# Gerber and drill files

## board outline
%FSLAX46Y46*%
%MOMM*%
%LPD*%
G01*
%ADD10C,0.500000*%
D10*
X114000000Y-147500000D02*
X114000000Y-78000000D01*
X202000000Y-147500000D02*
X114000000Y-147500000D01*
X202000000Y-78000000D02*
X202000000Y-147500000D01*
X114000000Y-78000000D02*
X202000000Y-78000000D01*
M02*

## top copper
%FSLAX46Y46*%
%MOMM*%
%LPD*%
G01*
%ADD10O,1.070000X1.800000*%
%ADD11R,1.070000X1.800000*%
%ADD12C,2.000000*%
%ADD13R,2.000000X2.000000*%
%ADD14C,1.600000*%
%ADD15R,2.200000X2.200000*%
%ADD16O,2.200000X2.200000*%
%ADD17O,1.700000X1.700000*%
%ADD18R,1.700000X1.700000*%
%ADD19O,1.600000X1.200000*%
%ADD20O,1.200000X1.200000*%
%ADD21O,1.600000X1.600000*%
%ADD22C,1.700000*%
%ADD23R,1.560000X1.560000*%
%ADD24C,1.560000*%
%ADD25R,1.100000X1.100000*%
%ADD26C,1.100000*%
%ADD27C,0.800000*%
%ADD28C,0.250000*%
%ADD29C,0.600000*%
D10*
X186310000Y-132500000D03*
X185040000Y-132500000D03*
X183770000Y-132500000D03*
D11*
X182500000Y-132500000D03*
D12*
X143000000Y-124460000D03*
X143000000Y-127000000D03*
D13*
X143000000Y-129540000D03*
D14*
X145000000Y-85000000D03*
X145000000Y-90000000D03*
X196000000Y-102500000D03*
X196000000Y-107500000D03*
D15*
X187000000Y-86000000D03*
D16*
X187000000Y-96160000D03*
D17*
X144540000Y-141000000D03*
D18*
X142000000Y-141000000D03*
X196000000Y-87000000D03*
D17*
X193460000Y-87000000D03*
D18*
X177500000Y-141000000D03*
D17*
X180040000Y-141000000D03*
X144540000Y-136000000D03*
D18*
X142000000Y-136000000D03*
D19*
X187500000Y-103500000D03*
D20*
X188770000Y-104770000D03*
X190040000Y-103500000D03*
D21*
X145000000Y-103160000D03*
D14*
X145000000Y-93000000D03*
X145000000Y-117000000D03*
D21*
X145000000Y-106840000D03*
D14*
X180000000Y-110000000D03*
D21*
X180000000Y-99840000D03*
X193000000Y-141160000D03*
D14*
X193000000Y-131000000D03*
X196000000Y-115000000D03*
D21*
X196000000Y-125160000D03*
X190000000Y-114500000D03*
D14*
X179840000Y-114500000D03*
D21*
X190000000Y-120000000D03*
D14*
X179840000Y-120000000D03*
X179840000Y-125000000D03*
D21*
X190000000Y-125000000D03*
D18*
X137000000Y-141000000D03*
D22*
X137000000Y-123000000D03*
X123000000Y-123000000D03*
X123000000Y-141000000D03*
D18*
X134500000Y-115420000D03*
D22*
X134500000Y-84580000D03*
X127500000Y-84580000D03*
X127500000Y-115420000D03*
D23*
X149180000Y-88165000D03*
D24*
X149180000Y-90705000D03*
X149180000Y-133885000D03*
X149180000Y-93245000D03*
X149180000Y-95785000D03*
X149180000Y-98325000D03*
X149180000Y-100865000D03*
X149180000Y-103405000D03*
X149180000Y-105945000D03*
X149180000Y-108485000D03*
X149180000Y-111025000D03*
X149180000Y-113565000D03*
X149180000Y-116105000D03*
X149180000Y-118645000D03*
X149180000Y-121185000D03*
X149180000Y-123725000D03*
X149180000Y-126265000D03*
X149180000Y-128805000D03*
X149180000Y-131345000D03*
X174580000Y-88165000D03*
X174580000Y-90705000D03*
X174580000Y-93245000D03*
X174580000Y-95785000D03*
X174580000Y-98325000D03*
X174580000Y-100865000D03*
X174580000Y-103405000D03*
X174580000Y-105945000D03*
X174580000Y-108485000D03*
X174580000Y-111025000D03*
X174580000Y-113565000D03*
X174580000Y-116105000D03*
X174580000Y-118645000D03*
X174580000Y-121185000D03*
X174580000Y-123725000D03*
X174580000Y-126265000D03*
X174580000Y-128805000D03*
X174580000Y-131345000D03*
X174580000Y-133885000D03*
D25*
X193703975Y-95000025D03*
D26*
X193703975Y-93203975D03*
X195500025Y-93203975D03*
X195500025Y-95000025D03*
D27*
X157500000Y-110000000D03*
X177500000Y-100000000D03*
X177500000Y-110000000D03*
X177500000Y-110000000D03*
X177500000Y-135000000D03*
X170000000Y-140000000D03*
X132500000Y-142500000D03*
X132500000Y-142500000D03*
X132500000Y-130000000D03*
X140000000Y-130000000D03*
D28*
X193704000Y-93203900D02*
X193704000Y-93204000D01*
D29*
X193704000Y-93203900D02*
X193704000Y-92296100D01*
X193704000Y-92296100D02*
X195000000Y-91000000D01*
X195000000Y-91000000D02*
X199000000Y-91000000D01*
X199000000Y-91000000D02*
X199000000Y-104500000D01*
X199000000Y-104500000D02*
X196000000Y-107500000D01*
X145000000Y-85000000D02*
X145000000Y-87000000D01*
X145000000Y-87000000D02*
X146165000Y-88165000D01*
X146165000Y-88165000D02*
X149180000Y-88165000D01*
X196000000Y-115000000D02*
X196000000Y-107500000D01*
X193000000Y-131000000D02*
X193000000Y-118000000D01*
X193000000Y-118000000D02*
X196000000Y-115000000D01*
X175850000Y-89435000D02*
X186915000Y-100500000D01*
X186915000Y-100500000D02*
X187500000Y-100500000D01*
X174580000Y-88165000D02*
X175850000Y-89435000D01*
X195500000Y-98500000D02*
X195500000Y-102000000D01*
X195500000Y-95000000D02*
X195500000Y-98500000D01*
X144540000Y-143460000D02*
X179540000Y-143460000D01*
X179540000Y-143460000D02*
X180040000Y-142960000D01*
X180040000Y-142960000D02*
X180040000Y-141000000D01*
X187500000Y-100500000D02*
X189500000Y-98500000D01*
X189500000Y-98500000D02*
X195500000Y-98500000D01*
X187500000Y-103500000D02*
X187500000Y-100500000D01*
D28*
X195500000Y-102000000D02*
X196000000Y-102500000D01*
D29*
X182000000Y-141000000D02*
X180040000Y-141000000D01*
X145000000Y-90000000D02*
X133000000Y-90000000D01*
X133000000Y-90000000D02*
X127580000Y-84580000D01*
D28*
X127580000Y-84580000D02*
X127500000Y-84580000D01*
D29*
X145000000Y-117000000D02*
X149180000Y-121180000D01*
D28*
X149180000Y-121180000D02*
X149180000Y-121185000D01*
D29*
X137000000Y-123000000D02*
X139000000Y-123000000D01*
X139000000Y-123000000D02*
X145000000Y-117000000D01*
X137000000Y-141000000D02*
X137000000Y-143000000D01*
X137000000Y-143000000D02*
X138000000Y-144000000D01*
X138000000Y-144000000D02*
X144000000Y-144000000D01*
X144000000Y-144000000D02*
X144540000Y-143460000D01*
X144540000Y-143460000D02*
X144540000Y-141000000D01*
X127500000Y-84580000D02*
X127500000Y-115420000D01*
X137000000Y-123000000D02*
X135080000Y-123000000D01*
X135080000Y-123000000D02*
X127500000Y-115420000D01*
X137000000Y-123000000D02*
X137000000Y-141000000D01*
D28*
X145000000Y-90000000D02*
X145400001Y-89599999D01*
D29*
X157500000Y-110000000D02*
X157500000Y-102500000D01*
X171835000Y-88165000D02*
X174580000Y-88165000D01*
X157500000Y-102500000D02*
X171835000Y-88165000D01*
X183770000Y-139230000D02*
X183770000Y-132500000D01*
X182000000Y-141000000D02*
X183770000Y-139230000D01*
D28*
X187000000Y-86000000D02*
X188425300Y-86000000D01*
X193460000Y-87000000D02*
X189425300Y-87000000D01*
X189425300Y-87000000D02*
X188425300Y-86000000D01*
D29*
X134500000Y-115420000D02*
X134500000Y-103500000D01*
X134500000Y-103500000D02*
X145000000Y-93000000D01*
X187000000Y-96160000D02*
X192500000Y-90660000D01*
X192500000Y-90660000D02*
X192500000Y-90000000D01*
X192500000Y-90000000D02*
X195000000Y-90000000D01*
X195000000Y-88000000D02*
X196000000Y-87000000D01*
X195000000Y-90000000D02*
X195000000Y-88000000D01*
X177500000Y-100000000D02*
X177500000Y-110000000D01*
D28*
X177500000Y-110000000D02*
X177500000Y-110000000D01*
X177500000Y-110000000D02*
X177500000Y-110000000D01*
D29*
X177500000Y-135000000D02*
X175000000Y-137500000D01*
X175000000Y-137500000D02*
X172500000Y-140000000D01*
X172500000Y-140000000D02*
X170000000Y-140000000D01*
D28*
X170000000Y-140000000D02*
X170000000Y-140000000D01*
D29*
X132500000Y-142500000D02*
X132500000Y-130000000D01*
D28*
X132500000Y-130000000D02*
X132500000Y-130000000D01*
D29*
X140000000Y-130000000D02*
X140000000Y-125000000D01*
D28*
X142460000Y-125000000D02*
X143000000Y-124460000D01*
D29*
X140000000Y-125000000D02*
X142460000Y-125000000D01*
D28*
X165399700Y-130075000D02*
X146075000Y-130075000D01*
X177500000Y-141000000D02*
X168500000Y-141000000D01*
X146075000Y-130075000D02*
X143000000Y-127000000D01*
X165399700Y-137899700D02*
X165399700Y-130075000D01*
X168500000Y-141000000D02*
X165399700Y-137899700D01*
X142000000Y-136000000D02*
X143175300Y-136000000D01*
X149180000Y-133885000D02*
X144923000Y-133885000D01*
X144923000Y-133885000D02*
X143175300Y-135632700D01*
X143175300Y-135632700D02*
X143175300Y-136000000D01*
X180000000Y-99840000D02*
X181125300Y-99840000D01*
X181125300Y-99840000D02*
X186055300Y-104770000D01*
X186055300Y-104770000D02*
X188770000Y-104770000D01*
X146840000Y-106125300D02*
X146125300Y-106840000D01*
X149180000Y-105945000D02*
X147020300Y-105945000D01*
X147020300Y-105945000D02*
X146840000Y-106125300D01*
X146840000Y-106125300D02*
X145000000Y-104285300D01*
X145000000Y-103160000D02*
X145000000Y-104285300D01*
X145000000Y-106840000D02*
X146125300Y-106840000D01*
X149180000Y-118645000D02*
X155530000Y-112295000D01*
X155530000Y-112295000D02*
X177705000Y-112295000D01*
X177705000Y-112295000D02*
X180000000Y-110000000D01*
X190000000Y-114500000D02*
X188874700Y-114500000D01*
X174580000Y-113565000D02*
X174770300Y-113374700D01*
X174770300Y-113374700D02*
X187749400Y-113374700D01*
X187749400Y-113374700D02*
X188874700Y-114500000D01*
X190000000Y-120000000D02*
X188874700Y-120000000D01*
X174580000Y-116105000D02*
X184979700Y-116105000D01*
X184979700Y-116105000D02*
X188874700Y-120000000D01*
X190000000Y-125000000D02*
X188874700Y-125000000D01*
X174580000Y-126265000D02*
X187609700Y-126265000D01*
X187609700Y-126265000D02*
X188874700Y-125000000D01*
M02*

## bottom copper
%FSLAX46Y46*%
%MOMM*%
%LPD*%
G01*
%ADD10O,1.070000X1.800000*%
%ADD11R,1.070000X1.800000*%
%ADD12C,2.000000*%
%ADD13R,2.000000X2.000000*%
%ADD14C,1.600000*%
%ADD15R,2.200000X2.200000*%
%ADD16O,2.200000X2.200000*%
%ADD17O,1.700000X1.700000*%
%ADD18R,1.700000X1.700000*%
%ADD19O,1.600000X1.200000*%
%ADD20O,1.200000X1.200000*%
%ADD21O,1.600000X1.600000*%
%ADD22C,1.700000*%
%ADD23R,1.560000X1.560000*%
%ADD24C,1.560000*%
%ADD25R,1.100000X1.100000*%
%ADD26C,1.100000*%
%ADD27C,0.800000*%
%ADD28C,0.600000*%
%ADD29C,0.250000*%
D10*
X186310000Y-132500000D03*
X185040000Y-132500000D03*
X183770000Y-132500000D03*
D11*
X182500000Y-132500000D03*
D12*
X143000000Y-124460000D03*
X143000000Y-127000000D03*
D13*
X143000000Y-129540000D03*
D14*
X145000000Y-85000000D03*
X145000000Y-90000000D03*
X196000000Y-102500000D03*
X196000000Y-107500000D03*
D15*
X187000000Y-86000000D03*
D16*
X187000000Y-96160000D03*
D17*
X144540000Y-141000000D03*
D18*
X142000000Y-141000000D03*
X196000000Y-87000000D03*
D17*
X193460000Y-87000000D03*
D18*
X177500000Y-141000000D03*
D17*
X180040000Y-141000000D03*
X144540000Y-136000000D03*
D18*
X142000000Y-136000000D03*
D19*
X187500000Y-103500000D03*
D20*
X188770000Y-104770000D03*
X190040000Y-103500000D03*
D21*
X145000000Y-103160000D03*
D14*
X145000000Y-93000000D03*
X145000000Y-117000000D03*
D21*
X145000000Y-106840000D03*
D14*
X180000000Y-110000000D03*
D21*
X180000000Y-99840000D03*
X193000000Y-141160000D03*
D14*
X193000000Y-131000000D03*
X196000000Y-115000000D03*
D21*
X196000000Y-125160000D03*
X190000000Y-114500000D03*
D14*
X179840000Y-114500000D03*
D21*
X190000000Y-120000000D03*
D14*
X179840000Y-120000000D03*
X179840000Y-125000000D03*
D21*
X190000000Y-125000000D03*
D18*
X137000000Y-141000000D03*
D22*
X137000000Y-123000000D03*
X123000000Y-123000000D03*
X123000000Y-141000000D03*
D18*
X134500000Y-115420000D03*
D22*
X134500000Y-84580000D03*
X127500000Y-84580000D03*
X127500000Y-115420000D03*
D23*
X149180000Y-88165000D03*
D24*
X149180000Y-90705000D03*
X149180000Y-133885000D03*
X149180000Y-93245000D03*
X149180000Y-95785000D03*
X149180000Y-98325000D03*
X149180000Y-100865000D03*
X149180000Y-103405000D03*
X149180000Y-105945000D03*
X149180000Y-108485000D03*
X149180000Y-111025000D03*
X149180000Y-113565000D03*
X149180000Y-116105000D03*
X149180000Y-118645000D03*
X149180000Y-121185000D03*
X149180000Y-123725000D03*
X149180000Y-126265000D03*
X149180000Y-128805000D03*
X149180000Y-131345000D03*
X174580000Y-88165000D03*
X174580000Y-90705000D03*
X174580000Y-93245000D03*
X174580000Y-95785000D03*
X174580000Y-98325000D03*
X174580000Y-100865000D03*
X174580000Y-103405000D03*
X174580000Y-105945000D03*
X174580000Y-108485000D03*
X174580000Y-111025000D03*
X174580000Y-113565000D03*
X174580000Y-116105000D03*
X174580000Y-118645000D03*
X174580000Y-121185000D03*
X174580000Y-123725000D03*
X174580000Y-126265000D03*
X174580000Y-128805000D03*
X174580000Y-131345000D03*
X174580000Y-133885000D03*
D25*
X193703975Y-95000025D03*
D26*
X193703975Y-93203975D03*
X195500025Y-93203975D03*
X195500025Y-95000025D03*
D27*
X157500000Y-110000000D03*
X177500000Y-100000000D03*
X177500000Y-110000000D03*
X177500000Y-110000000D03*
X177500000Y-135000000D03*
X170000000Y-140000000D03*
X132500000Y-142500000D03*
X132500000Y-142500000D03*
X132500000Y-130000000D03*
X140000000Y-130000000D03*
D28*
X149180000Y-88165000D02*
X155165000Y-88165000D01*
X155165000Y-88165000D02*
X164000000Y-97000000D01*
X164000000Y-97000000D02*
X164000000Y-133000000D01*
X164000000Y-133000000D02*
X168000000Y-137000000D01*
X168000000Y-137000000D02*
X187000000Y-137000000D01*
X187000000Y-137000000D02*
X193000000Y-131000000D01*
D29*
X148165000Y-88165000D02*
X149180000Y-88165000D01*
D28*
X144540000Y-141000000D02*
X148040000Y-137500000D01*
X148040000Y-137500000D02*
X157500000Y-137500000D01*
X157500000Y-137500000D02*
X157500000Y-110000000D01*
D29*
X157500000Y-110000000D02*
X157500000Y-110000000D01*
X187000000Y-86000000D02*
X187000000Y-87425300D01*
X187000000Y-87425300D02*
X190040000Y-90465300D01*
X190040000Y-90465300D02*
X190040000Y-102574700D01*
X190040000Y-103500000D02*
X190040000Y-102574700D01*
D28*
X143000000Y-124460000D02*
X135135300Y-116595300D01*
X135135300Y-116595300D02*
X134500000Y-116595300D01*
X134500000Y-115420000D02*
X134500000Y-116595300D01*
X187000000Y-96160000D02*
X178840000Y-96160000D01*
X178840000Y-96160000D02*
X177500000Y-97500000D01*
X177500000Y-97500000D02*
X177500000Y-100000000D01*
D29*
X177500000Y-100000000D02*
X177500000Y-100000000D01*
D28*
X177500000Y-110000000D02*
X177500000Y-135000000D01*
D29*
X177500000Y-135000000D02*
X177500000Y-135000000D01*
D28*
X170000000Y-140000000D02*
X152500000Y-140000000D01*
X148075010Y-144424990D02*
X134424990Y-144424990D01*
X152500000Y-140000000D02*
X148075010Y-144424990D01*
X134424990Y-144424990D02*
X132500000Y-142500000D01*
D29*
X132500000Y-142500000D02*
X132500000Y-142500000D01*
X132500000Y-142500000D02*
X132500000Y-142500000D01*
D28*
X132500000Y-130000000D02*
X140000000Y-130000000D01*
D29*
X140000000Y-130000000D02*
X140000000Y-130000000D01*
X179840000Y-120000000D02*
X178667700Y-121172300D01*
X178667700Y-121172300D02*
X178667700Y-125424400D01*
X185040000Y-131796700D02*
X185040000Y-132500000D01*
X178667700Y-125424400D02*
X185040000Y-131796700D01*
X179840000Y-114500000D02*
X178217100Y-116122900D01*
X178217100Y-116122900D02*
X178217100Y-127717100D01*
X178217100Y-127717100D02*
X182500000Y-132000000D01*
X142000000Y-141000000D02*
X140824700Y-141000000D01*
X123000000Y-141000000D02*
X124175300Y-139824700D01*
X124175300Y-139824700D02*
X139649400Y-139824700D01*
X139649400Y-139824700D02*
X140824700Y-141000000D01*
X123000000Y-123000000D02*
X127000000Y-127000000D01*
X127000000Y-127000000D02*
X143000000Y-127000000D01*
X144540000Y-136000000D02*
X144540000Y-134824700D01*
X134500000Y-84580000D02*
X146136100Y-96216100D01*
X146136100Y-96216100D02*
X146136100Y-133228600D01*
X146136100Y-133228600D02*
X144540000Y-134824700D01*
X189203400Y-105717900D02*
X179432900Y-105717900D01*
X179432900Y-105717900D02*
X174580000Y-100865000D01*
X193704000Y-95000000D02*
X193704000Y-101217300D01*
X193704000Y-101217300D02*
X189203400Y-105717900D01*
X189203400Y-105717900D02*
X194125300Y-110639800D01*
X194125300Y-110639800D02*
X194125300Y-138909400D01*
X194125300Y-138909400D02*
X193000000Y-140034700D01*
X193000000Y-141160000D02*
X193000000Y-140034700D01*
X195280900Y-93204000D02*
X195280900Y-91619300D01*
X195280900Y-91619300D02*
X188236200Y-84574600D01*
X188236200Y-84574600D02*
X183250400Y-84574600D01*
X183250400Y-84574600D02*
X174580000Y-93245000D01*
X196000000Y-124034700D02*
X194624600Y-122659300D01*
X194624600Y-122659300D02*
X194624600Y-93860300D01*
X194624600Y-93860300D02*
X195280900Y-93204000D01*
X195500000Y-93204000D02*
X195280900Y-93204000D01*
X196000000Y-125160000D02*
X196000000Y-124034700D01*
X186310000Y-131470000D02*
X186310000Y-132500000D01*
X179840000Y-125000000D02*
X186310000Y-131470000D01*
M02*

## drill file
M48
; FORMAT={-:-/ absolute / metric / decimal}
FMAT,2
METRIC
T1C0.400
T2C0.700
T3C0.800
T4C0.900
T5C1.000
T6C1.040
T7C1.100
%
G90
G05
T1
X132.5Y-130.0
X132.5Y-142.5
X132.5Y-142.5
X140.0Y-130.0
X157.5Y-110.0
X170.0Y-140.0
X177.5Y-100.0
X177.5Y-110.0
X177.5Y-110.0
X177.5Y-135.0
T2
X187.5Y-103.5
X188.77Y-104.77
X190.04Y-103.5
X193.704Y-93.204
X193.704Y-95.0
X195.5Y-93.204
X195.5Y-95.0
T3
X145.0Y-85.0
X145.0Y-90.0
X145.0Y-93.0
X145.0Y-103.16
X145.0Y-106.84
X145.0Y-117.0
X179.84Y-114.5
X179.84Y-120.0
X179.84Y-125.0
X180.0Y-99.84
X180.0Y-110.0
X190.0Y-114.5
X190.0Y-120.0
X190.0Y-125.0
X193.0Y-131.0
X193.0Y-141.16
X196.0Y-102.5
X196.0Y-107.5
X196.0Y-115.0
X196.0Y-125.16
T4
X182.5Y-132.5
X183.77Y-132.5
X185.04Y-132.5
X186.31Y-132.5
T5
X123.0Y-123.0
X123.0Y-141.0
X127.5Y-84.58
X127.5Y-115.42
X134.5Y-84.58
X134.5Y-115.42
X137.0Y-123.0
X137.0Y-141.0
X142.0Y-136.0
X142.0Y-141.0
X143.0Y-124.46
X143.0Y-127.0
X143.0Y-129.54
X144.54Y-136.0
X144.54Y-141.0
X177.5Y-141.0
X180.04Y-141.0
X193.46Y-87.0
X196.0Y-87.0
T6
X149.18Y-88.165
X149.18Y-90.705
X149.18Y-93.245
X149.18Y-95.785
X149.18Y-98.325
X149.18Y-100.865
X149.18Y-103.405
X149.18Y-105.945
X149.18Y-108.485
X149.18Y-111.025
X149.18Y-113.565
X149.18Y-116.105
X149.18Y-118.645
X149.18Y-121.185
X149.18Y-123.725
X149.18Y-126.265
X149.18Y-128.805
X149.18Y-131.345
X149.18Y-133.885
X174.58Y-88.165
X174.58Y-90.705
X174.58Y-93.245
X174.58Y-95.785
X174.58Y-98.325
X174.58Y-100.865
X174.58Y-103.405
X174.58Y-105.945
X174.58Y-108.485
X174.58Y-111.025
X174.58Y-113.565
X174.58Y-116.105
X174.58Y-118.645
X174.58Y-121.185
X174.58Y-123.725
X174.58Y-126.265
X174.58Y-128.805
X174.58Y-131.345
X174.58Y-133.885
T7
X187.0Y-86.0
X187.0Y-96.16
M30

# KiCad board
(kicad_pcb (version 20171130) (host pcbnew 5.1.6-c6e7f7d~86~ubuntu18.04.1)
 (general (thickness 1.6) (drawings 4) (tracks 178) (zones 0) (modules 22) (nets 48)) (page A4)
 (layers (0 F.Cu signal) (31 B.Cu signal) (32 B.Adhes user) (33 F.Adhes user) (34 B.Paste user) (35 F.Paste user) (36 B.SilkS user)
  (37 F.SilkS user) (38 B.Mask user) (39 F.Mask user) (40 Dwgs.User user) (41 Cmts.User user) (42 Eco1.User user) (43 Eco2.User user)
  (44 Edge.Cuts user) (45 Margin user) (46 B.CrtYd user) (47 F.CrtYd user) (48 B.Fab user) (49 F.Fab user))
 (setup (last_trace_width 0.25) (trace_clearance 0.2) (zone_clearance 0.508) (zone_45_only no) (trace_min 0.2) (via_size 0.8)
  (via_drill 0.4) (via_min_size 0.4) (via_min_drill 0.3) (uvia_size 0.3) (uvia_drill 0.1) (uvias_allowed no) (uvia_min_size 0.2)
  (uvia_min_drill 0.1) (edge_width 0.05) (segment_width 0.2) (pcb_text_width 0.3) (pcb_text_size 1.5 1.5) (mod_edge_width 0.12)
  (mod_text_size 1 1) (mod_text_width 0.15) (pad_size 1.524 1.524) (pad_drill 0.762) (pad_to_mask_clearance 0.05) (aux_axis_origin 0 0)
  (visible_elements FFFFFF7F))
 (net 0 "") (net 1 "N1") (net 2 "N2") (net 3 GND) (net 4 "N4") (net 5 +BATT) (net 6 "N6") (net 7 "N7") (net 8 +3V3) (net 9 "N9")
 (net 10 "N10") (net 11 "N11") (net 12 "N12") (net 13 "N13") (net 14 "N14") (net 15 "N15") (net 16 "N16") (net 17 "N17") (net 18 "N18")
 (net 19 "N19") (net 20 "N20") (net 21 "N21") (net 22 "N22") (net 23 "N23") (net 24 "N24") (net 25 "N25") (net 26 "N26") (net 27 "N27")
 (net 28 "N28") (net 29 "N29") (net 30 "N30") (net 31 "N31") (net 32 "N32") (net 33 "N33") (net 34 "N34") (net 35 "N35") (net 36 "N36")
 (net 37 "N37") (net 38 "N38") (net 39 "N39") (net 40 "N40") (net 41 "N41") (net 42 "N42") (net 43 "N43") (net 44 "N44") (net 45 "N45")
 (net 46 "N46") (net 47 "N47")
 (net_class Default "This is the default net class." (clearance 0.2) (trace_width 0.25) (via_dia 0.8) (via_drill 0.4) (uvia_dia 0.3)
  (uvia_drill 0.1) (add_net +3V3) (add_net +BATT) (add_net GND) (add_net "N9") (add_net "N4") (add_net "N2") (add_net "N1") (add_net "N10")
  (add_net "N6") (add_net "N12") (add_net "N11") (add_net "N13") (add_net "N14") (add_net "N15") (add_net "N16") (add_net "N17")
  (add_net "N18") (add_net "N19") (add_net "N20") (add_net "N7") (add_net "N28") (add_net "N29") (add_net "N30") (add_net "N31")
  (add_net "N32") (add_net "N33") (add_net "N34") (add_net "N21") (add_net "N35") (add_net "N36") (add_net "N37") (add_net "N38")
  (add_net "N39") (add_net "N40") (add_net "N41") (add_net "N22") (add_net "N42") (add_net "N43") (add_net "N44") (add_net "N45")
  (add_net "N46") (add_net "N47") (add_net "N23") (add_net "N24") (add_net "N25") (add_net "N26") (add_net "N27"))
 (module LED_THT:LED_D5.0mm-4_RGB (layer F.Cu) (at 182.5 132.5)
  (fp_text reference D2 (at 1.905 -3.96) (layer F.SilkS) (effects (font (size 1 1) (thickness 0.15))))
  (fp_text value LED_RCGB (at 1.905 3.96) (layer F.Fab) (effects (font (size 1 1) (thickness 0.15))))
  (pad 4 thru_hole oval (at 3.81 0) (size 1.07 1.8) (drill 0.9) (layers *.Cu *.Mask) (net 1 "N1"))
  (pad 3 thru_hole oval (at 2.54 0) (size 1.07 1.8) (drill 0.9) (layers *.Cu *.Mask) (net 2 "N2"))
  (pad 2 thru_hole oval (at 1.27 0) (size 1.07 1.8) (drill 0.9) (layers *.Cu *.Mask) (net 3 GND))
  (pad 1 thru_hole rect (at 0 0) (size 1.07 1.8) (drill 0.9) (layers *.Cu *.Mask) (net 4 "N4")))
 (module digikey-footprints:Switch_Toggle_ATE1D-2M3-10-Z (layer F.Cu) (at 143 127 90)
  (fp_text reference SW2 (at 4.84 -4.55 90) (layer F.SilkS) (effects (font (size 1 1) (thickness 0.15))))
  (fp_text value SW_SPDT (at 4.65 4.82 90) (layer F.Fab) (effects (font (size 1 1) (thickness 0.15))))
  (pad 3 thru_hole circle (at 2.54 0 90) (size 2 2) (drill 1) (layers *.Cu *.Mask) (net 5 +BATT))
  (pad 2 thru_hole circle (at 0 0 90) (size 2 2) (drill 1) (layers *.Cu *.Mask) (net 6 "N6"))
  (pad 1 thru_hole rect (at -2.54 0 90) (size 2 2) (drill 1) (layers *.Cu *.Mask) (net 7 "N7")))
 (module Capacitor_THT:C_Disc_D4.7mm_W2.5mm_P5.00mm (layer F.Cu) (at 145 85 270)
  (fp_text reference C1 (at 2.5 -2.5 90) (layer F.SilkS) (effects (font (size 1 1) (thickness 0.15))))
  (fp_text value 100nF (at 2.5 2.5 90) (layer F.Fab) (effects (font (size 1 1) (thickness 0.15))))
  (pad 1 thru_hole circle (at 0 0 270) (size 1.6 1.6) (drill 0.8) (layers *.Cu *.Mask) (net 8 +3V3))
  (pad 2 thru_hole circle (at 5 0 270) (size 1.6 1.6) (drill 0.8) (layers *.Cu *.Mask) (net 3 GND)))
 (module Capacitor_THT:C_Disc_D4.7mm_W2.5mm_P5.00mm (layer F.Cu) (at 196 107.5 90)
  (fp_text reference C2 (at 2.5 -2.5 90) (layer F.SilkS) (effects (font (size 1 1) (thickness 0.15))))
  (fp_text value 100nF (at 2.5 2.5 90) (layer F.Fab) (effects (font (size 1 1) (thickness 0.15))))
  (pad 2 thru_hole circle (at 5 0 90) (size 1.6 1.6) (drill 0.8) (layers *.Cu *.Mask) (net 3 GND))
  (pad 1 thru_hole circle (at 0 0 90) (size 1.6 1.6) (drill 0.8) (layers *.Cu *.Mask) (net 8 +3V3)))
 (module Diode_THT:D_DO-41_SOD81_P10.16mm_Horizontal (layer F.Cu) (at 187 86 270)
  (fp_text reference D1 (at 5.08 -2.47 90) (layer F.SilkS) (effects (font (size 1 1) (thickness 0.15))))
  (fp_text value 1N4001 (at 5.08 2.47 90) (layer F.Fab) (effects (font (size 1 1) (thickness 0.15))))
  (pad 1 thru_hole rect (at 0 0 270) (size 2.2 2.2) (drill 1.1) (layers *.Cu *.Mask) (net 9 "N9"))
  (pad 2 thru_hole oval (at 10.16 0 270) (size 2.2 2.2) (drill 1.1) (layers *.Cu *.Mask) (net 5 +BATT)))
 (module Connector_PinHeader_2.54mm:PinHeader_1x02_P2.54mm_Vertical (layer F.Cu) (at 142 141 90)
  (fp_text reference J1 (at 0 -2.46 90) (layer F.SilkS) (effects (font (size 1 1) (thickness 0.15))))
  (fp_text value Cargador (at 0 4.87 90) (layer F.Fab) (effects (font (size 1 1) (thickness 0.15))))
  (pad 2 thru_hole oval (at 0 2.54 90) (size 1.7 1.7) (drill 1) (layers *.Cu *.Mask) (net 3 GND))
  (pad 1 thru_hole rect (at 0 0 90) (size 1.7 1.7) (drill 1) (layers *.Cu *.Mask) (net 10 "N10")))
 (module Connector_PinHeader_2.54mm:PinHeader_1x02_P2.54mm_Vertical (layer F.Cu) (at 196 87 270)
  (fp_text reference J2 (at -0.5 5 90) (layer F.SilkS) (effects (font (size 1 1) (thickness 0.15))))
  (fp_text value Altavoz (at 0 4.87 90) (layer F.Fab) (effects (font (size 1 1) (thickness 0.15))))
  (pad 1 thru_hole rect (at 0 0 270) (size 1.7 1.7) (drill 1) (layers *.Cu *.Mask) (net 5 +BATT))
  (pad 2 thru_hole oval (at 0 2.54 270) (size 1.7 1.7) (drill 1) (layers *.Cu *.Mask) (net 9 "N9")))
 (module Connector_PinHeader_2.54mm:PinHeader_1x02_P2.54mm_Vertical (layer F.Cu) (at 177.5 141 90)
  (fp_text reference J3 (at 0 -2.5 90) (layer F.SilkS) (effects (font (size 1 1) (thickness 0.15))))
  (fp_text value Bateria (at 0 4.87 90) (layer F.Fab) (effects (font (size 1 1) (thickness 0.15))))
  (pad 1 thru_hole rect (at 0 0 90) (size 1.7 1.7) (drill 1) (layers *.Cu *.Mask) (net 6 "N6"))
  (pad 2 thru_hole oval (at 0 2.54 90) (size 1.7 1.7) (drill 1) (layers *.Cu *.Mask) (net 3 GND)))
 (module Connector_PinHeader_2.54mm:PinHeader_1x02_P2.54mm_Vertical (layer F.Cu) (at 142 136 90)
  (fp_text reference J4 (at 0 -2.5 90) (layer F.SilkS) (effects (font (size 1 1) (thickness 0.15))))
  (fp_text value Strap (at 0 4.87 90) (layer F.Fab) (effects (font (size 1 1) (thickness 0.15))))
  (pad 2 thru_hole oval (at 0 2.54 90) (size 1.7 1.7) (drill 1) (layers *.Cu *.Mask) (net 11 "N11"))
  (pad 1 thru_hole rect (at 0 0 90) (size 1.7 1.7) (drill 1) (layers *.Cu *.Mask) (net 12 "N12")))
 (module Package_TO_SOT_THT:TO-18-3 (layer F.Cu) (at 187.5 103.5)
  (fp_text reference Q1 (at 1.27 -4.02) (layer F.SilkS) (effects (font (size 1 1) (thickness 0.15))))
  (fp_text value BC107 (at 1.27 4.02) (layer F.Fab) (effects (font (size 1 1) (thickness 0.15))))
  (pad 1 thru_hole oval (at 0 0) (size 1.6 1.2) (drill 0.7) (layers *.Cu *.Mask) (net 3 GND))
  (pad 2 thru_hole oval (at 1.27 1.27) (size 1.2 1.2) (drill 0.7) (layers *.Cu *.Mask) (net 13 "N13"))
  (pad 3 thru_hole oval (at 2.54 0) (size 1.2 1.2) (drill 0.7) (layers *.Cu *.Mask) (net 9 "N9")))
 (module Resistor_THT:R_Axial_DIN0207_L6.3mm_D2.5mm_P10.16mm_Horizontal (layer F.Cu) (at 145 93 270)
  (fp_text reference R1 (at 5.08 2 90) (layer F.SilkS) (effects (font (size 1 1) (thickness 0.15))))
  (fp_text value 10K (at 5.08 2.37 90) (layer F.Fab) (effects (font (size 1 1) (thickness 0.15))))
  (pad 2 thru_hole oval (at 10.16 0 270) (size 1.6 1.6) (drill 0.8) (layers *.Cu *.Mask) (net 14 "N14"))
  (pad 1 thru_hole circle (at 0 0 270) (size 1.6 1.6) (drill 0.8) (layers *.Cu *.Mask) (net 5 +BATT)))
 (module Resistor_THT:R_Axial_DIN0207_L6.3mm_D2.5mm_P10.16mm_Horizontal (layer F.Cu) (at 145 117 90)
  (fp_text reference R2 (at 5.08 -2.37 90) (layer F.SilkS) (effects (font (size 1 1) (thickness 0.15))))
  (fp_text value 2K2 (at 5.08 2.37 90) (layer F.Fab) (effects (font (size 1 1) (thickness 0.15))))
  (pad 1 thru_hole circle (at 0 0 90) (size 1.6 1.6) (drill 0.8) (layers *.Cu *.Mask) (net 3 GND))
  (pad 2 thru_hole oval (at 10.16 0 90) (size 1.6 1.6) (drill 0.8) (layers *.Cu *.Mask) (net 14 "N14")))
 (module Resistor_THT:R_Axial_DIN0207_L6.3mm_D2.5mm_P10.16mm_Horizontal (layer F.Cu) (at 180 110 90)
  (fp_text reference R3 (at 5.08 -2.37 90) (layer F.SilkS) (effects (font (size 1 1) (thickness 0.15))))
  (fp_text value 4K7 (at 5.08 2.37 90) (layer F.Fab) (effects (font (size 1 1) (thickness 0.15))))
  (pad 1 thru_hole circle (at 0 0 90) (size 1.6 1.6) (drill 0.8) (layers *.Cu *.Mask) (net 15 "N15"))
  (pad 2 thru_hole oval (at 10.16 0 90) (size 1.6 1.6) (drill 0.8) (layers *.Cu *.Mask) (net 13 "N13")))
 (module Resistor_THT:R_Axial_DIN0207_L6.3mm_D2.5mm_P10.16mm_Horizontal (layer F.Cu) (at 193 131 270)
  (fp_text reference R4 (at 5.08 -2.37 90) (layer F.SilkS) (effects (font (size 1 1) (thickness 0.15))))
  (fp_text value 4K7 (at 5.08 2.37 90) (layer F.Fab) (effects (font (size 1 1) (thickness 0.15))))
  (pad 2 thru_hole oval (at 10.16 0 270) (size 1.6 1.6) (drill 0.8) (layers *.Cu *.Mask) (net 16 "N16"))
  (pad 1 thru_hole circle (at 0 0 270) (size 1.6 1.6) (drill 0.8) (layers *.Cu *.Mask) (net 8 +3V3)))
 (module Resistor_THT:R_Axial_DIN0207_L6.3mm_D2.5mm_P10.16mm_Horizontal (layer F.Cu) (at 196 115 270)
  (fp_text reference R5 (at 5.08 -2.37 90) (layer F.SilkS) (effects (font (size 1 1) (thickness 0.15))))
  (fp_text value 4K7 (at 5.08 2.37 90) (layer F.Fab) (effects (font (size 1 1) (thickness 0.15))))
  (pad 1 thru_hole circle (at 0 0 270) (size 1.6 1.6) (drill 0.8) (layers *.Cu *.Mask) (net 8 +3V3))
  (pad 2 thru_hole oval (at 10.16 0 270) (size 1.6 1.6) (drill 0.8) (layers *.Cu *.Mask) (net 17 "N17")))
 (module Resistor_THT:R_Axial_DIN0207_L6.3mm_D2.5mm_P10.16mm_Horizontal (layer F.Cu) (at 179.84 114.5)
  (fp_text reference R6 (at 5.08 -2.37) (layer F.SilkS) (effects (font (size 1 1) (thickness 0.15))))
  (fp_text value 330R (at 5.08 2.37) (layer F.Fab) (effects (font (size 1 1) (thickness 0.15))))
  (pad 2 thru_hole oval (at 10.16 0) (size 1.6 1.6) (drill 0.8) (layers *.Cu *.Mask) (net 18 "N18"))
  (pad 1 thru_hole circle (at 0 0) (size 1.6 1.6) (drill 0.8) (layers *.Cu *.Mask) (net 4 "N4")))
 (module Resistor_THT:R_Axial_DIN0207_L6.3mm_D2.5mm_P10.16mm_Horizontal (layer F.Cu) (at 179.84 120)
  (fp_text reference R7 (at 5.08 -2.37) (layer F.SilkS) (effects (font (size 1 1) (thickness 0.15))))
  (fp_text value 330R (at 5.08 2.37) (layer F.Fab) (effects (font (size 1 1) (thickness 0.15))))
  (pad 2 thru_hole oval (at 10.16 0) (size 1.6 1.6) (drill 0.8) (layers *.Cu *.Mask) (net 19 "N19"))
  (pad 1 thru_hole circle (at 0 0) (size 1.6 1.6) (drill 0.8) (layers *.Cu *.Mask) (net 2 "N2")))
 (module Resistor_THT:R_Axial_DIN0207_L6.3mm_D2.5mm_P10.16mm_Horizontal (layer F.Cu) (at 179.84 125)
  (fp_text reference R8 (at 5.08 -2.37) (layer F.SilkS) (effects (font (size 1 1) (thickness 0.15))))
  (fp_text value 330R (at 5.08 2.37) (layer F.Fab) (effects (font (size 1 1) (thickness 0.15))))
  (pad 1 thru_hole circle (at 0 0) (size 1.6 1.6) (drill 0.8) (layers *.Cu *.Mask) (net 1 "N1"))
  (pad 2 thru_hole oval (at 10.16 0) (size 1.6 1.6) (drill 0.8) (layers *.Cu *.Mask) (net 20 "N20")))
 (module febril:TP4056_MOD (layer F.Cu) (at 130 132 90)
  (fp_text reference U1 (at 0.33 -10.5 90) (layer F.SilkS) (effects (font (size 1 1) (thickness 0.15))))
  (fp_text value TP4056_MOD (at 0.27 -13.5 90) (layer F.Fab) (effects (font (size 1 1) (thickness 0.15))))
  (pad 1 thru_hole rect (at -9 7 90) (size 1.7 1.7) (drill 1) (layers *.Cu *.Mask) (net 3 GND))
  (pad 2 thru_hole circle (at 9 7 90) (size 1.7 1.7) (drill 1) (layers *.Cu *.Mask) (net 3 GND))
  (pad 3 thru_hole circle (at 9 -7 90) (size 1.7 1.7) (drill 1) (layers *.Cu *.Mask) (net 6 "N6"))
  (pad 4 thru_hole circle (at -9 -7 90) (size 1.7 1.7) (drill 1) (layers *.Cu *.Mask) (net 10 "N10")))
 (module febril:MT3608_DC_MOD (layer F.Cu) (at 131 100 90)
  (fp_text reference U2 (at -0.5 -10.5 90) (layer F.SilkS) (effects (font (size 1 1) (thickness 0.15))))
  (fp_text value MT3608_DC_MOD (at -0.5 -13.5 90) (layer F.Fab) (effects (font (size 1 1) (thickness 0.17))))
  (pad 1 thru_hole rect (at -15.42 3.5 90) (size 1.7 1.7) (drill 1) (layers *.Cu *.Mask) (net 5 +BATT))
  (pad 2 thru_hole circle (at 15.42 3.5 90) (size 1.7 1.7) (drill 1) (layers *.Cu *.Mask) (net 11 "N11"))
  (pad 3 thru_hole circle (at 15.42 -3.5 90) (size 1.7 1.7) (drill 1) (layers *.Cu *.Mask) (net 3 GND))
  (pad 4 thru_hole circle (at -15.42 -3.5 90) (size 1.7 1.7) (drill 1) (layers *.Cu *.Mask) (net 3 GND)))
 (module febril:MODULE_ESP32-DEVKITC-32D (layer F.Cu) (at 161.88 107.925)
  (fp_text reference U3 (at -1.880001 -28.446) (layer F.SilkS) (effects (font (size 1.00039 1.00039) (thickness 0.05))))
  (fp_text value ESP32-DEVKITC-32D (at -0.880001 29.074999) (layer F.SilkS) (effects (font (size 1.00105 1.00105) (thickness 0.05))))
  (pad 1 thru_hole rect (at -12.7 -19.76) (size 1.56 1.56) (drill 1.04) (layers *.Cu *.Mask) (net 8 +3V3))
  (pad 2 thru_hole circle (at -12.7 -17.22) (size 1.56 1.56) (drill 1.04) (layers *.Cu *.Mask) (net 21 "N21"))
  (pad 19 thru_hole circle (at -12.7 25.96) (size 1.56 1.56) (drill 1.04) (layers *.Cu *.Mask) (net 12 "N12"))
  (pad 3 thru_hole circle (at -12.7 -14.68) (size 1.56 1.56) (drill 1.04) (layers *.Cu *.Mask) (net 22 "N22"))
  (pad 4 thru_hole circle (at -12.7 -12.14) (size 1.56 1.56) (drill 1.04) (layers *.Cu *.Mask) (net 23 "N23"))
  (pad 5 thru_hole circle (at -12.7 -9.6) (size 1.56 1.56) (drill 1.04) (layers *.Cu *.Mask) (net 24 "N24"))
  (pad 6 thru_hole circle (at -12.7 -7.06) (size 1.56 1.56) (drill 1.04) (layers *.Cu *.Mask) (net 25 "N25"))
  (pad 7 thru_hole circle (at -12.7 -4.52) (size 1.56 1.56) (drill 1.04) (layers *.Cu *.Mask) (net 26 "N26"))
  (pad 8 thru_hole circle (at -12.7 -1.98) (size 1.56 1.56) (drill 1.04) (layers *.Cu *.Mask) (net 14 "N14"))
  (pad 9 thru_hole circle (at -12.7 0.56) (size 1.56 1.56) (drill 1.04) (layers *.Cu *.Mask) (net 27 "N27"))
  (pad 10 thru_hole circle (at -12.7 3.1) (size 1.56 1.56) (drill 1.04) (layers *.Cu *.Mask) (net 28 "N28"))
  (pad 11 thru_hole circle (at -12.7 5.64) (size 1.56 1.56) (drill 1.04) (layers *.Cu *.Mask) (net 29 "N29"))
  (pad 12 thru_hole circle (at -12.7 8.18) (size 1.56 1.56) (drill 1.04) (layers *.Cu *.Mask) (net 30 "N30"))
  (pad 13 thru_hole circle (at -12.7 10.72) (size 1.56 1.56) (drill 1.04) (layers *.Cu *.Mask) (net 15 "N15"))
  (pad 14 thru_hole circle (at -12.7 13.26) (size 1.56 1.56) (drill 1.04) (layers *.Cu *.Mask) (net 3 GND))
  (pad 15 thru_hole circle (at -12.7 15.8) (size 1.56 1.56) (drill 1.04) (layers *.Cu *.Mask) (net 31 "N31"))
  (pad 16 thru_hole circle (at -12.7 18.34) (size 1.56 1.56) (drill 1.04) (layers *.Cu *.Mask) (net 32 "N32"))
  (pad 17 thru_hole circle (at -12.7 20.88) (size 1.56 1.56) (drill 1.04) (layers *.Cu *.Mask) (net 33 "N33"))
  (pad 18 thru_hole circle (at -12.7 23.42) (size 1.56 1.56) (drill 1.04) (layers *.Cu *.Mask) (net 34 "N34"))
  (pad 20 thru_hole circle (at 12.7 -19.76) (size 1.56 1.56) (drill 1.04) (layers *.Cu *.Mask) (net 3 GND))
  (pad 21 thru_hole circle (at 12.7 -17.22) (size 1.56 1.56) (drill 1.04) (layers *.Cu *.Mask) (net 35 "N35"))
  (pad 22 thru_hole circle (at 12.7 -14.68) (size 1.56 1.56) (drill 1.04) (layers *.Cu *.Mask) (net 17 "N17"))
  (pad 23 thru_hole circle (at 12.7 -12.14) (size 1.56 1.56) (drill 1.04) (layers *.Cu *.Mask) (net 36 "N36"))
  (pad 24 thru_hole circle (at 12.7 -9.6) (size 1.56 1.56) (drill 1.04) (layers *.Cu *.Mask) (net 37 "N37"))
  (pad 25 thru_hole circle (at 12.7 -7.06) (size 1.56 1.56) (drill 1.04) (layers *.Cu *.Mask) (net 16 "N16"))
  (pad 26 thru_hole circle (at 12.7 -4.52) (size 1.56 1.56) (drill 1.04) (layers *.Cu *.Mask) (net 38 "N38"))
  (pad 27 thru_hole circle (at 12.7 -1.98) (size 1.56 1.56) (drill 1.04) (layers *.Cu *.Mask) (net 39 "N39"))
  (pad 28 thru_hole circle (at 12.7 0.56) (size 1.56 1.56) (drill 1.04) (layers *.Cu *.Mask) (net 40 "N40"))
  (pad 29 thru_hole circle (at 12.7 3.1) (size 1.56 1.56) (drill 1.04) (layers *.Cu *.Mask) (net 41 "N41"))
  (pad 30 thru_hole circle (at 12.7 5.64) (size 1.56 1.56) (drill 1.04) (layers *.Cu *.Mask) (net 18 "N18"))
  (pad 31 thru_hole circle (at 12.7 8.18) (size 1.56 1.56) (drill 1.04) (layers *.Cu *.Mask) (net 19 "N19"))
  (pad 32 thru_hole circle (at 12.7 10.72) (size 1.56 1.56) (drill 1.04) (layers *.Cu *.Mask) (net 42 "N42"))
  (pad 33 thru_hole circle (at 12.7 13.26) (size 1.56 1.56) (drill 1.04) (layers *.Cu *.Mask) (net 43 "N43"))
  (pad 34 thru_hole circle (at 12.7 15.8) (size 1.56 1.56) (drill 1.04) (layers *.Cu *.Mask) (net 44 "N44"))
  (pad 35 thru_hole circle (at 12.7 18.34) (size 1.56 1.56) (drill 1.04) (layers *.Cu *.Mask) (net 20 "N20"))
  (pad 36 thru_hole circle (at 12.7 20.88) (size 1.56 1.56) (drill 1.04) (layers *.Cu *.Mask) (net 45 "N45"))
  (pad 37 thru_hole circle (at 12.7 23.42) (size 1.56 1.56) (drill 1.04) (layers *.Cu *.Mask) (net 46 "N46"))
  (pad 38 thru_hole circle (at 12.7 25.96) (size 1.56 1.56) (drill 1.04) (layers *.Cu *.Mask) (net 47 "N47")))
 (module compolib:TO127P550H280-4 (layer B.Cu) (at 194.602 94.102)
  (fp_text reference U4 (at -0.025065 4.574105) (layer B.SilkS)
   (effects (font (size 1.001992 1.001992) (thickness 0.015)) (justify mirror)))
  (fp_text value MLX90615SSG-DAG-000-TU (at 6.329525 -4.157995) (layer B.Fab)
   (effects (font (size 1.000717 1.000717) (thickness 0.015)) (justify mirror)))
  (pad 1 thru_hole rect (at -0.898025 0.898025) (size 1.1 1.1) (drill 0.7) (layers *.Cu *.Mask) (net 16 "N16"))
  (pad 2 thru_hole circle (at -0.898025 -0.898025) (size 1.1 1.1) (drill 0.7) (layers *.Cu *.Mask) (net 8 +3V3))
  (pad 3 thru_hole circle (at 0.898025 -0.898025) (size 1.1 1.1) (drill 0.7) (layers *.Cu *.Mask) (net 17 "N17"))
  (pad 4 thru_hole circle (at 0.898025 0.898025) (size 1.1 1.1) (drill 0.7) (layers *.Cu *.Mask) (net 3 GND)))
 (gr_line (start 114 147.5) (end 114 78) (layer Edge.Cuts) (width 0.5))
 (gr_line (start 202 147.5) (end 114 147.5) (layer Edge.Cuts) (width 0.5))
 (gr_line (start 202 78) (end 202 147.5) (layer Edge.Cuts) (width 0.5))
 (gr_line (start 114 78) (end 202 78) (layer Edge.Cuts) (width 0.5))
 (segment (start 193.704 93.2039) (end 193.704 93.204) (width 0.25) (layer F.Cu) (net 8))
 (segment (start 193.704 93.2039) (end 193.704 92.2961) (width 0.6) (layer F.Cu) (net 8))
 (segment (start 193.704 92.2961) (end 195 91) (width 0.6) (layer F.Cu) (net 8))
 (segment (start 195 91) (end 199 91) (width 0.6) (layer F.Cu) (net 8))
 (segment (start 199 91) (end 199 104.5) (width 0.6) (layer F.Cu) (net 8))
 (segment (start 199 104.5) (end 196 107.5) (width 0.6) (layer F.Cu) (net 8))
 (segment (start 149.18 88.165) (end 155.165 88.165) (width 0.6) (layer B.Cu) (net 8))
 (segment (start 155.165 88.165) (end 164 97) (width 0.6) (layer B.Cu) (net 8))
 (segment (start 164 97) (end 164 133) (width 0.6) (layer B.Cu) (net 8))
 (segment (start 164 133) (end 168 137) (width 0.6) (layer B.Cu) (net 8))
 (segment (start 168 137) (end 187 137) (width 0.6) (layer B.Cu) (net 8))
 (segment (start 187 137) (end 193 131) (width 0.6) (layer B.Cu) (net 8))
 (segment (start 145 85) (end 145 87) (width 0.6) (layer F.Cu) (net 8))
 (segment (start 145 87) (end 146.165 88.165) (width 0.6) (layer F.Cu) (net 8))
 (segment (start 146.165 88.165) (end 149.18 88.165) (width 0.6) (layer F.Cu) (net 8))
 (segment (start 196 115) (end 196 107.5) (width 0.6) (layer F.Cu) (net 8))
 (segment (start 193 131) (end 193 118) (width 0.6) (layer F.Cu) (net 8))
 (segment (start 193 118) (end 196 115) (width 0.6) (layer F.Cu) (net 8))
 (segment (start 148.165 88.165) (end 149.18 88.165) (width 0.25) (layer B.Cu) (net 8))
 (segment (start 175.85 89.435) (end 186.915 100.5) (width 0.6) (layer F.Cu) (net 3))
 (segment (start 186.915 100.5) (end 187.5 100.5) (width 0.6) (layer F.Cu) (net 3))
 (segment (start 174.58 88.165) (end 175.85 89.435) (width 0.6) (layer F.Cu) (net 3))
 (segment (start 195.5 98.5) (end 195.5 102) (width 0.6) (layer F.Cu) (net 3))
 (segment (start 195.5 95) (end 195.5 98.5) (width 0.6) (layer F.Cu) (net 3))
 (segment (start 144.54 143.46) (end 179.54 143.46) (width 0.6) (layer F.Cu) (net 3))
 (segment (start 179.54 143.46) (end 180.04 142.96) (width 0.6) (layer F.Cu) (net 3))
 (segment (start 180.04 142.96) (end 180.04 141) (width 0.6) (layer F.Cu) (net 3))
 (segment (start 187.5 100.5) (end 189.5 98.5) (width 0.6) (layer F.Cu) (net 3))
 (segment (start 189.5 98.5) (end 195.5 98.5) (width 0.6) (layer F.Cu) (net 3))
 (segment (start 187.5 103.5) (end 187.5 100.5) (width 0.6) (layer F.Cu) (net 3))
 (segment (start 195.5 102) (end 196 102.5) (width 0.25) (layer F.Cu) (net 3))
 (segment (start 182 141) (end 180.04 141) (width 0.6) (layer F.Cu) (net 3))
 (segment (start 145 90) (end 133 90) (width 0.6) (layer F.Cu) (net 3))
 (segment (start 133 90) (end 127.58 84.58) (width 0.6) (layer F.Cu) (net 3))
 (segment (start 127.58 84.58) (end 127.5 84.58) (width 0.25) (layer F.Cu) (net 3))
 (segment (start 145 117) (end 149.18 121.18) (width 0.6) (layer F.Cu) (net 3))
 (segment (start 149.18 121.18) (end 149.18 121.185) (width 0.25) (layer F.Cu) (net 3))
 (segment (start 137 123) (end 139 123) (width 0.6) (layer F.Cu) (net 3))
 (segment (start 139 123) (end 145 117) (width 0.6) (layer F.Cu) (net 3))
 (segment (start 137 141) (end 137 143) (width 0.6) (layer F.Cu) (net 3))
 (segment (start 137 143) (end 138 144) (width 0.6) (layer F.Cu) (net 3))
 (segment (start 138 144) (end 144 144) (width 0.6) (layer F.Cu) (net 3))
 (segment (start 144 144) (end 144.54 143.46) (width 0.6) (layer F.Cu) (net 3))
 (segment (start 144.54 143.46) (end 144.54 141) (width 0.6) (layer F.Cu) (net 3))
 (segment (start 127.5 84.58) (end 127.5 115.42) (width 0.6) (layer F.Cu) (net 3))
 (segment (start 137 123) (end 135.08 123) (width 0.6) (layer F.Cu) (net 3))
 (segment (start 135.08 123) (end 127.5 115.42) (width 0.6) (layer F.Cu) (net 3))
 (segment (start 137 123) (end 137 141) (width 0.6) (layer F.Cu) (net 3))
 (segment (start 145 90) (end 145.400001 89.599999) (width 0.25) (layer F.Cu) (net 3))
 (segment (start 144.54 141) (end 148.04 137.5) (width 0.6) (layer B.Cu) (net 3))
 (segment (start 148.04 137.5) (end 157.5 137.5) (width 0.6) (layer B.Cu) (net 3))
 (segment (start 157.5 137.5) (end 157.5 110) (width 0.6) (layer B.Cu) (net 3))
 (segment (start 157.5 110) (end 157.5 110) (width 0.25) (layer B.Cu) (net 3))
 (via (at 157.5 110) (size 0.8) (drill 0.4) (layers F.Cu B.Cu) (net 3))
 (segment (start 157.5 110) (end 157.5 102.5) (width 0.6) (layer F.Cu) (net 3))
 (segment (start 171.835 88.165) (end 174.58 88.165) (width 0.6) (layer F.Cu) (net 3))
 (segment (start 157.5 102.5) (end 171.835 88.165) (width 0.6) (layer F.Cu) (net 3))
 (segment (start 183.77 139.23) (end 183.77 132.5) (width 0.6) (layer F.Cu) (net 3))
 (segment (start 182 141) (end 183.77 139.23) (width 0.6) (layer F.Cu) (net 3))
 (segment (start 187 86) (end 187 87.4253) (width 0.25) (layer B.Cu) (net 9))
 (segment (start 187 87.4253) (end 190.04 90.4653) (width 0.25) (layer B.Cu) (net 9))
 (segment (start 190.04 90.4653) (end 190.04 102.5747) (width 0.25) (layer B.Cu) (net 9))
 (segment (start 190.04 103.5) (end 190.04 102.5747) (width 0.25) (layer B.Cu) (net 9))
 (segment (start 187 86) (end 188.4253 86) (width 0.25) (layer F.Cu) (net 9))
 (segment (start 193.46 87) (end 189.4253 87) (width 0.25) (layer F.Cu) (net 9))
 (segment (start 189.4253 87) (end 188.4253 86) (width 0.25) (layer F.Cu) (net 9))
 (segment (start 134.5 115.42) (end 134.5 103.5) (width 0.6) (layer F.Cu) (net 5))
 (segment (start 134.5 103.5) (end 145 93) (width 0.6) (layer F.Cu) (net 5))
 (segment (start 143 124.46) (end 135.1353 116.5953) (width 0.6) (layer B.Cu) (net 5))
 (segment (start 135.1353 116.5953) (end 134.5 116.5953) (width 0.6) (layer B.Cu) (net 5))
 (segment (start 134.5 115.42) (end 134.5 116.5953) (width 0.6) (layer B.Cu) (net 5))
 (segment (start 187 96.16) (end 192.5 90.66) (width 0.6) (layer F.Cu) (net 5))
 (segment (start 192.5 90.66) (end 192.5 90) (width 0.6) (layer F.Cu) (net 5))
 (segment (start 192.5 90) (end 195 90) (width 0.6) (layer F.Cu) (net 5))
 (segment (start 195 88) (end 196 87) (width 0.6) (layer F.Cu) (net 5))
 (segment (start 195 90) (end 195 88) (width 0.6) (layer F.Cu) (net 5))
 (segment (start 187 96.16) (end 178.84 96.16) (width 0.6) (layer B.Cu) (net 5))
 (segment (start 178.84 96.16) (end 177.5 97.5) (width 0.6) (layer B.Cu) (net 5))
 (segment (start 177.5 97.5) (end 177.5 100) (width 0.6) (layer B.Cu) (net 5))
 (segment (start 177.5 100) (end 177.5 100) (width 0.25) (layer B.Cu) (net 5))
 (via (at 177.5 100) (size 0.8) (drill 0.4) (layers F.Cu B.Cu) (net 5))
 (segment (start 177.5 100) (end 177.5 110) (width 0.6) (layer F.Cu) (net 5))
 (segment (start 177.5 110) (end 177.5 110) (width 0.25) (layer F.Cu) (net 5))
 (via (at 177.5 110) (size 0.8) (drill 0.4) (layers F.Cu B.Cu) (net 5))
 (segment (start 177.5 110) (end 177.5 110) (width 0.25) (layer F.Cu) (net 5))
 (via (at 177.5 110) (size 0.8) (drill 0.4) (layers F.Cu B.Cu) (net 5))
 (segment (start 177.5 110) (end 177.5 135) (width 0.6) (layer B.Cu) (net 5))
 (segment (start 177.5 135) (end 177.5 135) (width 0.25) (layer B.Cu) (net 5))
 (via (at 177.5 135) (size 0.8) (drill 0.4) (layers F.Cu B.Cu) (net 5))
 (segment (start 177.5 135) (end 175 137.5) (width 0.6) (layer F.Cu) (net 5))
 (segment (start 175 137.5) (end 172.5 140) (width 0.6) (layer F.Cu) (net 5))
 (segment (start 172.5 140) (end 170 140) (width 0.6) (layer F.Cu) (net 5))
 (segment (start 170 140) (end 170 140) (width 0.25) (layer F.Cu) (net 5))
 (via (at 170 140) (size 0.8) (drill 0.4) (layers F.Cu B.Cu) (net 5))
 (segment (start 170 140) (end 152.5 140) (width 0.6) (layer B.Cu) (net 5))
 (segment (start 148.07501 144.42499) (end 134.42499 144.42499) (width 0.6) (layer B.Cu) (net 5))
 (segment (start 152.5 140) (end 148.07501 144.42499) (width 0.6) (layer B.Cu) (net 5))
 (segment (start 134.42499 144.42499) (end 132.5 142.5) (width 0.6) (layer B.Cu) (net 5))
 (segment (start 132.5 142.5) (end 132.5 142.5) (width 0.25) (layer B.Cu) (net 5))
 (via (at 132.5 142.5) (size 0.8) (drill 0.4) (layers F.Cu B.Cu) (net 5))
 (segment (start 132.5 142.5) (end 132.5 142.5) (width 0.25) (layer B.Cu) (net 5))
 (via (at 132.5 142.5) (size 0.8) (drill 0.4) (layers F.Cu B.Cu) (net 5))
 (segment (start 132.5 142.5) (end 132.5 130) (width 0.6) (layer F.Cu) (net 5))
 (segment (start 132.5 130) (end 132.5 130) (width 0.25) (layer F.Cu) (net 5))
 (via (at 132.5 130) (size 0.8) (drill 0.4) (layers F.Cu B.Cu) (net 5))
 (segment (start 132.5 130) (end 140 130) (width 0.6) (layer B.Cu) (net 5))
 (segment (start 140 130) (end 140 130) (width 0.25) (layer B.Cu) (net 5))
 (via (at 140 130) (size 0.8) (drill 0.4) (layers F.Cu B.Cu) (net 5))
 (segment (start 140 130) (end 140 125) (width 0.6) (layer F.Cu) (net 5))
 (segment (start 142.46 125) (end 143 124.46) (width 0.25) (layer F.Cu) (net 5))
 (segment (start 140 125) (end 142.46 125) (width 0.6) (layer F.Cu) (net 5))
 (segment (start 179.84 120) (end 178.6677 121.1723) (width 0.25) (layer B.Cu) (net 2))
 (segment (start 178.6677 121.1723) (end 178.6677 125.4244) (width 0.25) (layer B.Cu) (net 2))
 (segment (start 185.04 131.7967) (end 185.04 132.5) (width 0.25) (layer B.Cu) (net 2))
 (segment (start 178.6677 125.4244) (end 185.04 131.7967) (width 0.25) (layer B.Cu) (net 2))
 (segment (start 179.84 114.5) (end 178.2171 116.1229) (width 0.25) (layer B.Cu) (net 4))
 (segment (start 178.2171 116.1229) (end 178.2171 127.7171) (width 0.25) (layer B.Cu) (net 4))
 (segment (start 178.2171 127.7171) (end 182.5 132) (width 0.25) (layer B.Cu) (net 4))
 (segment (start 142 141) (end 140.8247 141) (width 0.25) (layer B.Cu) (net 10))
 (segment (start 123 141) (end 124.1753 139.8247) (width 0.25) (layer B.Cu) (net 10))
 (segment (start 124.1753 139.8247) (end 139.6494 139.8247) (width 0.25) (layer B.Cu) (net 10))
 (segment (start 139.6494 139.8247) (end 140.8247 141) (width 0.25) (layer B.Cu) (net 10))
 (segment (start 123 123) (end 127 127) (width 0.25) (layer B.Cu) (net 6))
 (segment (start 127 127) (end 143 127) (width 0.25) (layer B.Cu) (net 6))
 (segment (start 165.3997 130.075) (end 146.075 130.075) (width 0.25) (layer F.Cu) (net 6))
 (segment (start 177.5 141) (end 168.5 141) (width 0.25) (layer F.Cu) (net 6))
 (segment (start 146.075 130.075) (end 143 127) (width 0.25) (layer F.Cu) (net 6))
 (segment (start 165.3997 137.8997) (end 165.3997 130.075) (width 0.25) (layer F.Cu) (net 6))
 (segment (start 168.5 141) (end 165.3997 137.8997) (width 0.25) (layer F.Cu) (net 6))
 (segment (start 144.54 136) (end 144.54 134.8247) (width 0.25) (layer B.Cu) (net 11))
 (segment (start 134.5 84.58) (end 146.1361 96.2161) (width 0.25) (layer B.Cu) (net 11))
 (segment (start 146.1361 96.2161) (end 146.1361 133.2286) (width 0.25) (layer B.Cu) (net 11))
 (segment (start 146.1361 133.2286) (end 144.54 134.8247) (width 0.25) (layer B.Cu) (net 11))
 (segment (start 142 136) (end 143.1753 136) (width 0.25) (layer F.Cu) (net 12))
 (segment (start 149.18 133.885) (end 144.923 133.885) (width 0.25) (layer F.Cu) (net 12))
 (segment (start 144.923 133.885) (end 143.1753 135.6327) (width 0.25) (layer F.Cu) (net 12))
 (segment (start 143.1753 135.6327) (end 143.1753 136) (width 0.25) (layer F.Cu) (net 12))
 (segment (start 180 99.84) (end 181.1253 99.84) (width 0.25) (layer F.Cu) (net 13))
 (segment (start 181.1253 99.84) (end 186.0553 104.77) (width 0.25) (layer F.Cu) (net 13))
 (segment (start 186.0553 104.77) (end 188.77 104.77) (width 0.25) (layer F.Cu) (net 13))
 (segment (start 146.84 106.1253) (end 146.1253 106.84) (width 0.25) (layer F.Cu) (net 14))
 (segment (start 149.18 105.945) (end 147.0203 105.945) (width 0.25) (layer F.Cu) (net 14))
 (segment (start 147.0203 105.945) (end 146.84 106.1253) (width 0.25) (layer F.Cu) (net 14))
 (segment (start 146.84 106.1253) (end 145 104.2853) (width 0.25) (layer F.Cu) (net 14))
 (segment (start 145 103.16) (end 145 104.2853) (width 0.25) (layer F.Cu) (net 14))
 (segment (start 145 106.84) (end 146.1253 106.84) (width 0.25) (layer F.Cu) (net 14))
 (segment (start 149.18 118.645) (end 155.53 112.295) (width 0.25) (layer F.Cu) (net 15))
 (segment (start 155.53 112.295) (end 177.705 112.295) (width 0.25) (layer F.Cu) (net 15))
 (segment (start 177.705 112.295) (end 180 110) (width 0.25) (layer F.Cu) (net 15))
 (segment (start 189.2034 105.7179) (end 179.4329 105.7179) (width 0.25) (layer B.Cu) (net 16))
 (segment (start 179.4329 105.7179) (end 174.58 100.865) (width 0.25) (layer B.Cu) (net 16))
 (segment (start 193.704 95) (end 193.704 101.2173) (width 0.25) (layer B.Cu) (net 16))
 (segment (start 193.704 101.2173) (end 189.2034 105.7179) (width 0.25) (layer B.Cu) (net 16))
 (segment (start 189.2034 105.7179) (end 194.1253 110.6398) (width 0.25) (layer B.Cu) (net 16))
 (segment (start 194.1253 110.6398) (end 194.1253 138.9094) (width 0.25) (layer B.Cu) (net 16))
 (segment (start 194.1253 138.9094) (end 193 140.0347) (width 0.25) (layer B.Cu) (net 16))
 (segment (start 193 141.16) (end 193 140.0347) (width 0.25) (layer B.Cu) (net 16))
 (segment (start 195.2809 93.204) (end 195.2809 91.6193) (width 0.25) (layer B.Cu) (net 17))
 (segment (start 195.2809 91.6193) (end 188.2362 84.5746) (width 0.25) (layer B.Cu) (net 17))
 (segment (start 188.2362 84.5746) (end 183.2504 84.5746) (width 0.25) (layer B.Cu) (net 17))
 (segment (start 183.2504 84.5746) (end 174.58 93.245) (width 0.25) (layer B.Cu) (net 17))
 (segment (start 196 124.0347) (end 194.6246 122.6593) (width 0.25) (layer B.Cu) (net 17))
 (segment (start 194.6246 122.6593) (end 194.6246 93.8603) (width 0.25) (layer B.Cu) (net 17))
 (segment (start 194.6246 93.8603) (end 195.2809 93.204) (width 0.25) (layer B.Cu) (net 17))
 (segment (start 195.5 93.204) (end 195.2809 93.204) (width 0.25) (layer B.Cu) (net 17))
 (segment (start 196 125.16) (end 196 124.0347) (width 0.25) (layer B.Cu) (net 17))
 (segment (start 190 114.5) (end 188.8747 114.5) (width 0.25) (layer F.Cu) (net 18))
 (segment (start 174.58 113.565) (end 174.7703 113.3747) (width 0.25) (layer F.Cu) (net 18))
 (segment (start 174.7703 113.3747) (end 187.7494 113.3747) (width 0.25) (layer F.Cu) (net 18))
 (segment (start 187.7494 113.3747) (end 188.8747 114.5) (width 0.25) (layer F.Cu) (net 18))
 (segment (start 190 120) (end 188.8747 120) (width 0.25) (layer F.Cu) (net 19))
 (segment (start 174.58 116.105) (end 184.9797 116.105) (width 0.25) (layer F.Cu) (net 19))
 (segment (start 184.9797 116.105) (end 188.8747 120) (width 0.25) (layer F.Cu) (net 19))
 (segment (start 190 125) (end 188.8747 125) (width 0.25) (layer F.Cu) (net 20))
 (segment (start 174.58 126.265) (end 187.6097 126.265) (width 0.25) (layer F.Cu) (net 20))
 (segment (start 187.6097 126.265) (end 188.8747 125) (width 0.25) (layer F.Cu) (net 20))
 (segment (start 186.31 131.47) (end 186.31 132.5) (width 0.25) (layer B.Cu) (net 1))
 (segment (start 179.84 125) (end 186.31 131.47) (width 0.25) (layer B.Cu) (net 1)))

